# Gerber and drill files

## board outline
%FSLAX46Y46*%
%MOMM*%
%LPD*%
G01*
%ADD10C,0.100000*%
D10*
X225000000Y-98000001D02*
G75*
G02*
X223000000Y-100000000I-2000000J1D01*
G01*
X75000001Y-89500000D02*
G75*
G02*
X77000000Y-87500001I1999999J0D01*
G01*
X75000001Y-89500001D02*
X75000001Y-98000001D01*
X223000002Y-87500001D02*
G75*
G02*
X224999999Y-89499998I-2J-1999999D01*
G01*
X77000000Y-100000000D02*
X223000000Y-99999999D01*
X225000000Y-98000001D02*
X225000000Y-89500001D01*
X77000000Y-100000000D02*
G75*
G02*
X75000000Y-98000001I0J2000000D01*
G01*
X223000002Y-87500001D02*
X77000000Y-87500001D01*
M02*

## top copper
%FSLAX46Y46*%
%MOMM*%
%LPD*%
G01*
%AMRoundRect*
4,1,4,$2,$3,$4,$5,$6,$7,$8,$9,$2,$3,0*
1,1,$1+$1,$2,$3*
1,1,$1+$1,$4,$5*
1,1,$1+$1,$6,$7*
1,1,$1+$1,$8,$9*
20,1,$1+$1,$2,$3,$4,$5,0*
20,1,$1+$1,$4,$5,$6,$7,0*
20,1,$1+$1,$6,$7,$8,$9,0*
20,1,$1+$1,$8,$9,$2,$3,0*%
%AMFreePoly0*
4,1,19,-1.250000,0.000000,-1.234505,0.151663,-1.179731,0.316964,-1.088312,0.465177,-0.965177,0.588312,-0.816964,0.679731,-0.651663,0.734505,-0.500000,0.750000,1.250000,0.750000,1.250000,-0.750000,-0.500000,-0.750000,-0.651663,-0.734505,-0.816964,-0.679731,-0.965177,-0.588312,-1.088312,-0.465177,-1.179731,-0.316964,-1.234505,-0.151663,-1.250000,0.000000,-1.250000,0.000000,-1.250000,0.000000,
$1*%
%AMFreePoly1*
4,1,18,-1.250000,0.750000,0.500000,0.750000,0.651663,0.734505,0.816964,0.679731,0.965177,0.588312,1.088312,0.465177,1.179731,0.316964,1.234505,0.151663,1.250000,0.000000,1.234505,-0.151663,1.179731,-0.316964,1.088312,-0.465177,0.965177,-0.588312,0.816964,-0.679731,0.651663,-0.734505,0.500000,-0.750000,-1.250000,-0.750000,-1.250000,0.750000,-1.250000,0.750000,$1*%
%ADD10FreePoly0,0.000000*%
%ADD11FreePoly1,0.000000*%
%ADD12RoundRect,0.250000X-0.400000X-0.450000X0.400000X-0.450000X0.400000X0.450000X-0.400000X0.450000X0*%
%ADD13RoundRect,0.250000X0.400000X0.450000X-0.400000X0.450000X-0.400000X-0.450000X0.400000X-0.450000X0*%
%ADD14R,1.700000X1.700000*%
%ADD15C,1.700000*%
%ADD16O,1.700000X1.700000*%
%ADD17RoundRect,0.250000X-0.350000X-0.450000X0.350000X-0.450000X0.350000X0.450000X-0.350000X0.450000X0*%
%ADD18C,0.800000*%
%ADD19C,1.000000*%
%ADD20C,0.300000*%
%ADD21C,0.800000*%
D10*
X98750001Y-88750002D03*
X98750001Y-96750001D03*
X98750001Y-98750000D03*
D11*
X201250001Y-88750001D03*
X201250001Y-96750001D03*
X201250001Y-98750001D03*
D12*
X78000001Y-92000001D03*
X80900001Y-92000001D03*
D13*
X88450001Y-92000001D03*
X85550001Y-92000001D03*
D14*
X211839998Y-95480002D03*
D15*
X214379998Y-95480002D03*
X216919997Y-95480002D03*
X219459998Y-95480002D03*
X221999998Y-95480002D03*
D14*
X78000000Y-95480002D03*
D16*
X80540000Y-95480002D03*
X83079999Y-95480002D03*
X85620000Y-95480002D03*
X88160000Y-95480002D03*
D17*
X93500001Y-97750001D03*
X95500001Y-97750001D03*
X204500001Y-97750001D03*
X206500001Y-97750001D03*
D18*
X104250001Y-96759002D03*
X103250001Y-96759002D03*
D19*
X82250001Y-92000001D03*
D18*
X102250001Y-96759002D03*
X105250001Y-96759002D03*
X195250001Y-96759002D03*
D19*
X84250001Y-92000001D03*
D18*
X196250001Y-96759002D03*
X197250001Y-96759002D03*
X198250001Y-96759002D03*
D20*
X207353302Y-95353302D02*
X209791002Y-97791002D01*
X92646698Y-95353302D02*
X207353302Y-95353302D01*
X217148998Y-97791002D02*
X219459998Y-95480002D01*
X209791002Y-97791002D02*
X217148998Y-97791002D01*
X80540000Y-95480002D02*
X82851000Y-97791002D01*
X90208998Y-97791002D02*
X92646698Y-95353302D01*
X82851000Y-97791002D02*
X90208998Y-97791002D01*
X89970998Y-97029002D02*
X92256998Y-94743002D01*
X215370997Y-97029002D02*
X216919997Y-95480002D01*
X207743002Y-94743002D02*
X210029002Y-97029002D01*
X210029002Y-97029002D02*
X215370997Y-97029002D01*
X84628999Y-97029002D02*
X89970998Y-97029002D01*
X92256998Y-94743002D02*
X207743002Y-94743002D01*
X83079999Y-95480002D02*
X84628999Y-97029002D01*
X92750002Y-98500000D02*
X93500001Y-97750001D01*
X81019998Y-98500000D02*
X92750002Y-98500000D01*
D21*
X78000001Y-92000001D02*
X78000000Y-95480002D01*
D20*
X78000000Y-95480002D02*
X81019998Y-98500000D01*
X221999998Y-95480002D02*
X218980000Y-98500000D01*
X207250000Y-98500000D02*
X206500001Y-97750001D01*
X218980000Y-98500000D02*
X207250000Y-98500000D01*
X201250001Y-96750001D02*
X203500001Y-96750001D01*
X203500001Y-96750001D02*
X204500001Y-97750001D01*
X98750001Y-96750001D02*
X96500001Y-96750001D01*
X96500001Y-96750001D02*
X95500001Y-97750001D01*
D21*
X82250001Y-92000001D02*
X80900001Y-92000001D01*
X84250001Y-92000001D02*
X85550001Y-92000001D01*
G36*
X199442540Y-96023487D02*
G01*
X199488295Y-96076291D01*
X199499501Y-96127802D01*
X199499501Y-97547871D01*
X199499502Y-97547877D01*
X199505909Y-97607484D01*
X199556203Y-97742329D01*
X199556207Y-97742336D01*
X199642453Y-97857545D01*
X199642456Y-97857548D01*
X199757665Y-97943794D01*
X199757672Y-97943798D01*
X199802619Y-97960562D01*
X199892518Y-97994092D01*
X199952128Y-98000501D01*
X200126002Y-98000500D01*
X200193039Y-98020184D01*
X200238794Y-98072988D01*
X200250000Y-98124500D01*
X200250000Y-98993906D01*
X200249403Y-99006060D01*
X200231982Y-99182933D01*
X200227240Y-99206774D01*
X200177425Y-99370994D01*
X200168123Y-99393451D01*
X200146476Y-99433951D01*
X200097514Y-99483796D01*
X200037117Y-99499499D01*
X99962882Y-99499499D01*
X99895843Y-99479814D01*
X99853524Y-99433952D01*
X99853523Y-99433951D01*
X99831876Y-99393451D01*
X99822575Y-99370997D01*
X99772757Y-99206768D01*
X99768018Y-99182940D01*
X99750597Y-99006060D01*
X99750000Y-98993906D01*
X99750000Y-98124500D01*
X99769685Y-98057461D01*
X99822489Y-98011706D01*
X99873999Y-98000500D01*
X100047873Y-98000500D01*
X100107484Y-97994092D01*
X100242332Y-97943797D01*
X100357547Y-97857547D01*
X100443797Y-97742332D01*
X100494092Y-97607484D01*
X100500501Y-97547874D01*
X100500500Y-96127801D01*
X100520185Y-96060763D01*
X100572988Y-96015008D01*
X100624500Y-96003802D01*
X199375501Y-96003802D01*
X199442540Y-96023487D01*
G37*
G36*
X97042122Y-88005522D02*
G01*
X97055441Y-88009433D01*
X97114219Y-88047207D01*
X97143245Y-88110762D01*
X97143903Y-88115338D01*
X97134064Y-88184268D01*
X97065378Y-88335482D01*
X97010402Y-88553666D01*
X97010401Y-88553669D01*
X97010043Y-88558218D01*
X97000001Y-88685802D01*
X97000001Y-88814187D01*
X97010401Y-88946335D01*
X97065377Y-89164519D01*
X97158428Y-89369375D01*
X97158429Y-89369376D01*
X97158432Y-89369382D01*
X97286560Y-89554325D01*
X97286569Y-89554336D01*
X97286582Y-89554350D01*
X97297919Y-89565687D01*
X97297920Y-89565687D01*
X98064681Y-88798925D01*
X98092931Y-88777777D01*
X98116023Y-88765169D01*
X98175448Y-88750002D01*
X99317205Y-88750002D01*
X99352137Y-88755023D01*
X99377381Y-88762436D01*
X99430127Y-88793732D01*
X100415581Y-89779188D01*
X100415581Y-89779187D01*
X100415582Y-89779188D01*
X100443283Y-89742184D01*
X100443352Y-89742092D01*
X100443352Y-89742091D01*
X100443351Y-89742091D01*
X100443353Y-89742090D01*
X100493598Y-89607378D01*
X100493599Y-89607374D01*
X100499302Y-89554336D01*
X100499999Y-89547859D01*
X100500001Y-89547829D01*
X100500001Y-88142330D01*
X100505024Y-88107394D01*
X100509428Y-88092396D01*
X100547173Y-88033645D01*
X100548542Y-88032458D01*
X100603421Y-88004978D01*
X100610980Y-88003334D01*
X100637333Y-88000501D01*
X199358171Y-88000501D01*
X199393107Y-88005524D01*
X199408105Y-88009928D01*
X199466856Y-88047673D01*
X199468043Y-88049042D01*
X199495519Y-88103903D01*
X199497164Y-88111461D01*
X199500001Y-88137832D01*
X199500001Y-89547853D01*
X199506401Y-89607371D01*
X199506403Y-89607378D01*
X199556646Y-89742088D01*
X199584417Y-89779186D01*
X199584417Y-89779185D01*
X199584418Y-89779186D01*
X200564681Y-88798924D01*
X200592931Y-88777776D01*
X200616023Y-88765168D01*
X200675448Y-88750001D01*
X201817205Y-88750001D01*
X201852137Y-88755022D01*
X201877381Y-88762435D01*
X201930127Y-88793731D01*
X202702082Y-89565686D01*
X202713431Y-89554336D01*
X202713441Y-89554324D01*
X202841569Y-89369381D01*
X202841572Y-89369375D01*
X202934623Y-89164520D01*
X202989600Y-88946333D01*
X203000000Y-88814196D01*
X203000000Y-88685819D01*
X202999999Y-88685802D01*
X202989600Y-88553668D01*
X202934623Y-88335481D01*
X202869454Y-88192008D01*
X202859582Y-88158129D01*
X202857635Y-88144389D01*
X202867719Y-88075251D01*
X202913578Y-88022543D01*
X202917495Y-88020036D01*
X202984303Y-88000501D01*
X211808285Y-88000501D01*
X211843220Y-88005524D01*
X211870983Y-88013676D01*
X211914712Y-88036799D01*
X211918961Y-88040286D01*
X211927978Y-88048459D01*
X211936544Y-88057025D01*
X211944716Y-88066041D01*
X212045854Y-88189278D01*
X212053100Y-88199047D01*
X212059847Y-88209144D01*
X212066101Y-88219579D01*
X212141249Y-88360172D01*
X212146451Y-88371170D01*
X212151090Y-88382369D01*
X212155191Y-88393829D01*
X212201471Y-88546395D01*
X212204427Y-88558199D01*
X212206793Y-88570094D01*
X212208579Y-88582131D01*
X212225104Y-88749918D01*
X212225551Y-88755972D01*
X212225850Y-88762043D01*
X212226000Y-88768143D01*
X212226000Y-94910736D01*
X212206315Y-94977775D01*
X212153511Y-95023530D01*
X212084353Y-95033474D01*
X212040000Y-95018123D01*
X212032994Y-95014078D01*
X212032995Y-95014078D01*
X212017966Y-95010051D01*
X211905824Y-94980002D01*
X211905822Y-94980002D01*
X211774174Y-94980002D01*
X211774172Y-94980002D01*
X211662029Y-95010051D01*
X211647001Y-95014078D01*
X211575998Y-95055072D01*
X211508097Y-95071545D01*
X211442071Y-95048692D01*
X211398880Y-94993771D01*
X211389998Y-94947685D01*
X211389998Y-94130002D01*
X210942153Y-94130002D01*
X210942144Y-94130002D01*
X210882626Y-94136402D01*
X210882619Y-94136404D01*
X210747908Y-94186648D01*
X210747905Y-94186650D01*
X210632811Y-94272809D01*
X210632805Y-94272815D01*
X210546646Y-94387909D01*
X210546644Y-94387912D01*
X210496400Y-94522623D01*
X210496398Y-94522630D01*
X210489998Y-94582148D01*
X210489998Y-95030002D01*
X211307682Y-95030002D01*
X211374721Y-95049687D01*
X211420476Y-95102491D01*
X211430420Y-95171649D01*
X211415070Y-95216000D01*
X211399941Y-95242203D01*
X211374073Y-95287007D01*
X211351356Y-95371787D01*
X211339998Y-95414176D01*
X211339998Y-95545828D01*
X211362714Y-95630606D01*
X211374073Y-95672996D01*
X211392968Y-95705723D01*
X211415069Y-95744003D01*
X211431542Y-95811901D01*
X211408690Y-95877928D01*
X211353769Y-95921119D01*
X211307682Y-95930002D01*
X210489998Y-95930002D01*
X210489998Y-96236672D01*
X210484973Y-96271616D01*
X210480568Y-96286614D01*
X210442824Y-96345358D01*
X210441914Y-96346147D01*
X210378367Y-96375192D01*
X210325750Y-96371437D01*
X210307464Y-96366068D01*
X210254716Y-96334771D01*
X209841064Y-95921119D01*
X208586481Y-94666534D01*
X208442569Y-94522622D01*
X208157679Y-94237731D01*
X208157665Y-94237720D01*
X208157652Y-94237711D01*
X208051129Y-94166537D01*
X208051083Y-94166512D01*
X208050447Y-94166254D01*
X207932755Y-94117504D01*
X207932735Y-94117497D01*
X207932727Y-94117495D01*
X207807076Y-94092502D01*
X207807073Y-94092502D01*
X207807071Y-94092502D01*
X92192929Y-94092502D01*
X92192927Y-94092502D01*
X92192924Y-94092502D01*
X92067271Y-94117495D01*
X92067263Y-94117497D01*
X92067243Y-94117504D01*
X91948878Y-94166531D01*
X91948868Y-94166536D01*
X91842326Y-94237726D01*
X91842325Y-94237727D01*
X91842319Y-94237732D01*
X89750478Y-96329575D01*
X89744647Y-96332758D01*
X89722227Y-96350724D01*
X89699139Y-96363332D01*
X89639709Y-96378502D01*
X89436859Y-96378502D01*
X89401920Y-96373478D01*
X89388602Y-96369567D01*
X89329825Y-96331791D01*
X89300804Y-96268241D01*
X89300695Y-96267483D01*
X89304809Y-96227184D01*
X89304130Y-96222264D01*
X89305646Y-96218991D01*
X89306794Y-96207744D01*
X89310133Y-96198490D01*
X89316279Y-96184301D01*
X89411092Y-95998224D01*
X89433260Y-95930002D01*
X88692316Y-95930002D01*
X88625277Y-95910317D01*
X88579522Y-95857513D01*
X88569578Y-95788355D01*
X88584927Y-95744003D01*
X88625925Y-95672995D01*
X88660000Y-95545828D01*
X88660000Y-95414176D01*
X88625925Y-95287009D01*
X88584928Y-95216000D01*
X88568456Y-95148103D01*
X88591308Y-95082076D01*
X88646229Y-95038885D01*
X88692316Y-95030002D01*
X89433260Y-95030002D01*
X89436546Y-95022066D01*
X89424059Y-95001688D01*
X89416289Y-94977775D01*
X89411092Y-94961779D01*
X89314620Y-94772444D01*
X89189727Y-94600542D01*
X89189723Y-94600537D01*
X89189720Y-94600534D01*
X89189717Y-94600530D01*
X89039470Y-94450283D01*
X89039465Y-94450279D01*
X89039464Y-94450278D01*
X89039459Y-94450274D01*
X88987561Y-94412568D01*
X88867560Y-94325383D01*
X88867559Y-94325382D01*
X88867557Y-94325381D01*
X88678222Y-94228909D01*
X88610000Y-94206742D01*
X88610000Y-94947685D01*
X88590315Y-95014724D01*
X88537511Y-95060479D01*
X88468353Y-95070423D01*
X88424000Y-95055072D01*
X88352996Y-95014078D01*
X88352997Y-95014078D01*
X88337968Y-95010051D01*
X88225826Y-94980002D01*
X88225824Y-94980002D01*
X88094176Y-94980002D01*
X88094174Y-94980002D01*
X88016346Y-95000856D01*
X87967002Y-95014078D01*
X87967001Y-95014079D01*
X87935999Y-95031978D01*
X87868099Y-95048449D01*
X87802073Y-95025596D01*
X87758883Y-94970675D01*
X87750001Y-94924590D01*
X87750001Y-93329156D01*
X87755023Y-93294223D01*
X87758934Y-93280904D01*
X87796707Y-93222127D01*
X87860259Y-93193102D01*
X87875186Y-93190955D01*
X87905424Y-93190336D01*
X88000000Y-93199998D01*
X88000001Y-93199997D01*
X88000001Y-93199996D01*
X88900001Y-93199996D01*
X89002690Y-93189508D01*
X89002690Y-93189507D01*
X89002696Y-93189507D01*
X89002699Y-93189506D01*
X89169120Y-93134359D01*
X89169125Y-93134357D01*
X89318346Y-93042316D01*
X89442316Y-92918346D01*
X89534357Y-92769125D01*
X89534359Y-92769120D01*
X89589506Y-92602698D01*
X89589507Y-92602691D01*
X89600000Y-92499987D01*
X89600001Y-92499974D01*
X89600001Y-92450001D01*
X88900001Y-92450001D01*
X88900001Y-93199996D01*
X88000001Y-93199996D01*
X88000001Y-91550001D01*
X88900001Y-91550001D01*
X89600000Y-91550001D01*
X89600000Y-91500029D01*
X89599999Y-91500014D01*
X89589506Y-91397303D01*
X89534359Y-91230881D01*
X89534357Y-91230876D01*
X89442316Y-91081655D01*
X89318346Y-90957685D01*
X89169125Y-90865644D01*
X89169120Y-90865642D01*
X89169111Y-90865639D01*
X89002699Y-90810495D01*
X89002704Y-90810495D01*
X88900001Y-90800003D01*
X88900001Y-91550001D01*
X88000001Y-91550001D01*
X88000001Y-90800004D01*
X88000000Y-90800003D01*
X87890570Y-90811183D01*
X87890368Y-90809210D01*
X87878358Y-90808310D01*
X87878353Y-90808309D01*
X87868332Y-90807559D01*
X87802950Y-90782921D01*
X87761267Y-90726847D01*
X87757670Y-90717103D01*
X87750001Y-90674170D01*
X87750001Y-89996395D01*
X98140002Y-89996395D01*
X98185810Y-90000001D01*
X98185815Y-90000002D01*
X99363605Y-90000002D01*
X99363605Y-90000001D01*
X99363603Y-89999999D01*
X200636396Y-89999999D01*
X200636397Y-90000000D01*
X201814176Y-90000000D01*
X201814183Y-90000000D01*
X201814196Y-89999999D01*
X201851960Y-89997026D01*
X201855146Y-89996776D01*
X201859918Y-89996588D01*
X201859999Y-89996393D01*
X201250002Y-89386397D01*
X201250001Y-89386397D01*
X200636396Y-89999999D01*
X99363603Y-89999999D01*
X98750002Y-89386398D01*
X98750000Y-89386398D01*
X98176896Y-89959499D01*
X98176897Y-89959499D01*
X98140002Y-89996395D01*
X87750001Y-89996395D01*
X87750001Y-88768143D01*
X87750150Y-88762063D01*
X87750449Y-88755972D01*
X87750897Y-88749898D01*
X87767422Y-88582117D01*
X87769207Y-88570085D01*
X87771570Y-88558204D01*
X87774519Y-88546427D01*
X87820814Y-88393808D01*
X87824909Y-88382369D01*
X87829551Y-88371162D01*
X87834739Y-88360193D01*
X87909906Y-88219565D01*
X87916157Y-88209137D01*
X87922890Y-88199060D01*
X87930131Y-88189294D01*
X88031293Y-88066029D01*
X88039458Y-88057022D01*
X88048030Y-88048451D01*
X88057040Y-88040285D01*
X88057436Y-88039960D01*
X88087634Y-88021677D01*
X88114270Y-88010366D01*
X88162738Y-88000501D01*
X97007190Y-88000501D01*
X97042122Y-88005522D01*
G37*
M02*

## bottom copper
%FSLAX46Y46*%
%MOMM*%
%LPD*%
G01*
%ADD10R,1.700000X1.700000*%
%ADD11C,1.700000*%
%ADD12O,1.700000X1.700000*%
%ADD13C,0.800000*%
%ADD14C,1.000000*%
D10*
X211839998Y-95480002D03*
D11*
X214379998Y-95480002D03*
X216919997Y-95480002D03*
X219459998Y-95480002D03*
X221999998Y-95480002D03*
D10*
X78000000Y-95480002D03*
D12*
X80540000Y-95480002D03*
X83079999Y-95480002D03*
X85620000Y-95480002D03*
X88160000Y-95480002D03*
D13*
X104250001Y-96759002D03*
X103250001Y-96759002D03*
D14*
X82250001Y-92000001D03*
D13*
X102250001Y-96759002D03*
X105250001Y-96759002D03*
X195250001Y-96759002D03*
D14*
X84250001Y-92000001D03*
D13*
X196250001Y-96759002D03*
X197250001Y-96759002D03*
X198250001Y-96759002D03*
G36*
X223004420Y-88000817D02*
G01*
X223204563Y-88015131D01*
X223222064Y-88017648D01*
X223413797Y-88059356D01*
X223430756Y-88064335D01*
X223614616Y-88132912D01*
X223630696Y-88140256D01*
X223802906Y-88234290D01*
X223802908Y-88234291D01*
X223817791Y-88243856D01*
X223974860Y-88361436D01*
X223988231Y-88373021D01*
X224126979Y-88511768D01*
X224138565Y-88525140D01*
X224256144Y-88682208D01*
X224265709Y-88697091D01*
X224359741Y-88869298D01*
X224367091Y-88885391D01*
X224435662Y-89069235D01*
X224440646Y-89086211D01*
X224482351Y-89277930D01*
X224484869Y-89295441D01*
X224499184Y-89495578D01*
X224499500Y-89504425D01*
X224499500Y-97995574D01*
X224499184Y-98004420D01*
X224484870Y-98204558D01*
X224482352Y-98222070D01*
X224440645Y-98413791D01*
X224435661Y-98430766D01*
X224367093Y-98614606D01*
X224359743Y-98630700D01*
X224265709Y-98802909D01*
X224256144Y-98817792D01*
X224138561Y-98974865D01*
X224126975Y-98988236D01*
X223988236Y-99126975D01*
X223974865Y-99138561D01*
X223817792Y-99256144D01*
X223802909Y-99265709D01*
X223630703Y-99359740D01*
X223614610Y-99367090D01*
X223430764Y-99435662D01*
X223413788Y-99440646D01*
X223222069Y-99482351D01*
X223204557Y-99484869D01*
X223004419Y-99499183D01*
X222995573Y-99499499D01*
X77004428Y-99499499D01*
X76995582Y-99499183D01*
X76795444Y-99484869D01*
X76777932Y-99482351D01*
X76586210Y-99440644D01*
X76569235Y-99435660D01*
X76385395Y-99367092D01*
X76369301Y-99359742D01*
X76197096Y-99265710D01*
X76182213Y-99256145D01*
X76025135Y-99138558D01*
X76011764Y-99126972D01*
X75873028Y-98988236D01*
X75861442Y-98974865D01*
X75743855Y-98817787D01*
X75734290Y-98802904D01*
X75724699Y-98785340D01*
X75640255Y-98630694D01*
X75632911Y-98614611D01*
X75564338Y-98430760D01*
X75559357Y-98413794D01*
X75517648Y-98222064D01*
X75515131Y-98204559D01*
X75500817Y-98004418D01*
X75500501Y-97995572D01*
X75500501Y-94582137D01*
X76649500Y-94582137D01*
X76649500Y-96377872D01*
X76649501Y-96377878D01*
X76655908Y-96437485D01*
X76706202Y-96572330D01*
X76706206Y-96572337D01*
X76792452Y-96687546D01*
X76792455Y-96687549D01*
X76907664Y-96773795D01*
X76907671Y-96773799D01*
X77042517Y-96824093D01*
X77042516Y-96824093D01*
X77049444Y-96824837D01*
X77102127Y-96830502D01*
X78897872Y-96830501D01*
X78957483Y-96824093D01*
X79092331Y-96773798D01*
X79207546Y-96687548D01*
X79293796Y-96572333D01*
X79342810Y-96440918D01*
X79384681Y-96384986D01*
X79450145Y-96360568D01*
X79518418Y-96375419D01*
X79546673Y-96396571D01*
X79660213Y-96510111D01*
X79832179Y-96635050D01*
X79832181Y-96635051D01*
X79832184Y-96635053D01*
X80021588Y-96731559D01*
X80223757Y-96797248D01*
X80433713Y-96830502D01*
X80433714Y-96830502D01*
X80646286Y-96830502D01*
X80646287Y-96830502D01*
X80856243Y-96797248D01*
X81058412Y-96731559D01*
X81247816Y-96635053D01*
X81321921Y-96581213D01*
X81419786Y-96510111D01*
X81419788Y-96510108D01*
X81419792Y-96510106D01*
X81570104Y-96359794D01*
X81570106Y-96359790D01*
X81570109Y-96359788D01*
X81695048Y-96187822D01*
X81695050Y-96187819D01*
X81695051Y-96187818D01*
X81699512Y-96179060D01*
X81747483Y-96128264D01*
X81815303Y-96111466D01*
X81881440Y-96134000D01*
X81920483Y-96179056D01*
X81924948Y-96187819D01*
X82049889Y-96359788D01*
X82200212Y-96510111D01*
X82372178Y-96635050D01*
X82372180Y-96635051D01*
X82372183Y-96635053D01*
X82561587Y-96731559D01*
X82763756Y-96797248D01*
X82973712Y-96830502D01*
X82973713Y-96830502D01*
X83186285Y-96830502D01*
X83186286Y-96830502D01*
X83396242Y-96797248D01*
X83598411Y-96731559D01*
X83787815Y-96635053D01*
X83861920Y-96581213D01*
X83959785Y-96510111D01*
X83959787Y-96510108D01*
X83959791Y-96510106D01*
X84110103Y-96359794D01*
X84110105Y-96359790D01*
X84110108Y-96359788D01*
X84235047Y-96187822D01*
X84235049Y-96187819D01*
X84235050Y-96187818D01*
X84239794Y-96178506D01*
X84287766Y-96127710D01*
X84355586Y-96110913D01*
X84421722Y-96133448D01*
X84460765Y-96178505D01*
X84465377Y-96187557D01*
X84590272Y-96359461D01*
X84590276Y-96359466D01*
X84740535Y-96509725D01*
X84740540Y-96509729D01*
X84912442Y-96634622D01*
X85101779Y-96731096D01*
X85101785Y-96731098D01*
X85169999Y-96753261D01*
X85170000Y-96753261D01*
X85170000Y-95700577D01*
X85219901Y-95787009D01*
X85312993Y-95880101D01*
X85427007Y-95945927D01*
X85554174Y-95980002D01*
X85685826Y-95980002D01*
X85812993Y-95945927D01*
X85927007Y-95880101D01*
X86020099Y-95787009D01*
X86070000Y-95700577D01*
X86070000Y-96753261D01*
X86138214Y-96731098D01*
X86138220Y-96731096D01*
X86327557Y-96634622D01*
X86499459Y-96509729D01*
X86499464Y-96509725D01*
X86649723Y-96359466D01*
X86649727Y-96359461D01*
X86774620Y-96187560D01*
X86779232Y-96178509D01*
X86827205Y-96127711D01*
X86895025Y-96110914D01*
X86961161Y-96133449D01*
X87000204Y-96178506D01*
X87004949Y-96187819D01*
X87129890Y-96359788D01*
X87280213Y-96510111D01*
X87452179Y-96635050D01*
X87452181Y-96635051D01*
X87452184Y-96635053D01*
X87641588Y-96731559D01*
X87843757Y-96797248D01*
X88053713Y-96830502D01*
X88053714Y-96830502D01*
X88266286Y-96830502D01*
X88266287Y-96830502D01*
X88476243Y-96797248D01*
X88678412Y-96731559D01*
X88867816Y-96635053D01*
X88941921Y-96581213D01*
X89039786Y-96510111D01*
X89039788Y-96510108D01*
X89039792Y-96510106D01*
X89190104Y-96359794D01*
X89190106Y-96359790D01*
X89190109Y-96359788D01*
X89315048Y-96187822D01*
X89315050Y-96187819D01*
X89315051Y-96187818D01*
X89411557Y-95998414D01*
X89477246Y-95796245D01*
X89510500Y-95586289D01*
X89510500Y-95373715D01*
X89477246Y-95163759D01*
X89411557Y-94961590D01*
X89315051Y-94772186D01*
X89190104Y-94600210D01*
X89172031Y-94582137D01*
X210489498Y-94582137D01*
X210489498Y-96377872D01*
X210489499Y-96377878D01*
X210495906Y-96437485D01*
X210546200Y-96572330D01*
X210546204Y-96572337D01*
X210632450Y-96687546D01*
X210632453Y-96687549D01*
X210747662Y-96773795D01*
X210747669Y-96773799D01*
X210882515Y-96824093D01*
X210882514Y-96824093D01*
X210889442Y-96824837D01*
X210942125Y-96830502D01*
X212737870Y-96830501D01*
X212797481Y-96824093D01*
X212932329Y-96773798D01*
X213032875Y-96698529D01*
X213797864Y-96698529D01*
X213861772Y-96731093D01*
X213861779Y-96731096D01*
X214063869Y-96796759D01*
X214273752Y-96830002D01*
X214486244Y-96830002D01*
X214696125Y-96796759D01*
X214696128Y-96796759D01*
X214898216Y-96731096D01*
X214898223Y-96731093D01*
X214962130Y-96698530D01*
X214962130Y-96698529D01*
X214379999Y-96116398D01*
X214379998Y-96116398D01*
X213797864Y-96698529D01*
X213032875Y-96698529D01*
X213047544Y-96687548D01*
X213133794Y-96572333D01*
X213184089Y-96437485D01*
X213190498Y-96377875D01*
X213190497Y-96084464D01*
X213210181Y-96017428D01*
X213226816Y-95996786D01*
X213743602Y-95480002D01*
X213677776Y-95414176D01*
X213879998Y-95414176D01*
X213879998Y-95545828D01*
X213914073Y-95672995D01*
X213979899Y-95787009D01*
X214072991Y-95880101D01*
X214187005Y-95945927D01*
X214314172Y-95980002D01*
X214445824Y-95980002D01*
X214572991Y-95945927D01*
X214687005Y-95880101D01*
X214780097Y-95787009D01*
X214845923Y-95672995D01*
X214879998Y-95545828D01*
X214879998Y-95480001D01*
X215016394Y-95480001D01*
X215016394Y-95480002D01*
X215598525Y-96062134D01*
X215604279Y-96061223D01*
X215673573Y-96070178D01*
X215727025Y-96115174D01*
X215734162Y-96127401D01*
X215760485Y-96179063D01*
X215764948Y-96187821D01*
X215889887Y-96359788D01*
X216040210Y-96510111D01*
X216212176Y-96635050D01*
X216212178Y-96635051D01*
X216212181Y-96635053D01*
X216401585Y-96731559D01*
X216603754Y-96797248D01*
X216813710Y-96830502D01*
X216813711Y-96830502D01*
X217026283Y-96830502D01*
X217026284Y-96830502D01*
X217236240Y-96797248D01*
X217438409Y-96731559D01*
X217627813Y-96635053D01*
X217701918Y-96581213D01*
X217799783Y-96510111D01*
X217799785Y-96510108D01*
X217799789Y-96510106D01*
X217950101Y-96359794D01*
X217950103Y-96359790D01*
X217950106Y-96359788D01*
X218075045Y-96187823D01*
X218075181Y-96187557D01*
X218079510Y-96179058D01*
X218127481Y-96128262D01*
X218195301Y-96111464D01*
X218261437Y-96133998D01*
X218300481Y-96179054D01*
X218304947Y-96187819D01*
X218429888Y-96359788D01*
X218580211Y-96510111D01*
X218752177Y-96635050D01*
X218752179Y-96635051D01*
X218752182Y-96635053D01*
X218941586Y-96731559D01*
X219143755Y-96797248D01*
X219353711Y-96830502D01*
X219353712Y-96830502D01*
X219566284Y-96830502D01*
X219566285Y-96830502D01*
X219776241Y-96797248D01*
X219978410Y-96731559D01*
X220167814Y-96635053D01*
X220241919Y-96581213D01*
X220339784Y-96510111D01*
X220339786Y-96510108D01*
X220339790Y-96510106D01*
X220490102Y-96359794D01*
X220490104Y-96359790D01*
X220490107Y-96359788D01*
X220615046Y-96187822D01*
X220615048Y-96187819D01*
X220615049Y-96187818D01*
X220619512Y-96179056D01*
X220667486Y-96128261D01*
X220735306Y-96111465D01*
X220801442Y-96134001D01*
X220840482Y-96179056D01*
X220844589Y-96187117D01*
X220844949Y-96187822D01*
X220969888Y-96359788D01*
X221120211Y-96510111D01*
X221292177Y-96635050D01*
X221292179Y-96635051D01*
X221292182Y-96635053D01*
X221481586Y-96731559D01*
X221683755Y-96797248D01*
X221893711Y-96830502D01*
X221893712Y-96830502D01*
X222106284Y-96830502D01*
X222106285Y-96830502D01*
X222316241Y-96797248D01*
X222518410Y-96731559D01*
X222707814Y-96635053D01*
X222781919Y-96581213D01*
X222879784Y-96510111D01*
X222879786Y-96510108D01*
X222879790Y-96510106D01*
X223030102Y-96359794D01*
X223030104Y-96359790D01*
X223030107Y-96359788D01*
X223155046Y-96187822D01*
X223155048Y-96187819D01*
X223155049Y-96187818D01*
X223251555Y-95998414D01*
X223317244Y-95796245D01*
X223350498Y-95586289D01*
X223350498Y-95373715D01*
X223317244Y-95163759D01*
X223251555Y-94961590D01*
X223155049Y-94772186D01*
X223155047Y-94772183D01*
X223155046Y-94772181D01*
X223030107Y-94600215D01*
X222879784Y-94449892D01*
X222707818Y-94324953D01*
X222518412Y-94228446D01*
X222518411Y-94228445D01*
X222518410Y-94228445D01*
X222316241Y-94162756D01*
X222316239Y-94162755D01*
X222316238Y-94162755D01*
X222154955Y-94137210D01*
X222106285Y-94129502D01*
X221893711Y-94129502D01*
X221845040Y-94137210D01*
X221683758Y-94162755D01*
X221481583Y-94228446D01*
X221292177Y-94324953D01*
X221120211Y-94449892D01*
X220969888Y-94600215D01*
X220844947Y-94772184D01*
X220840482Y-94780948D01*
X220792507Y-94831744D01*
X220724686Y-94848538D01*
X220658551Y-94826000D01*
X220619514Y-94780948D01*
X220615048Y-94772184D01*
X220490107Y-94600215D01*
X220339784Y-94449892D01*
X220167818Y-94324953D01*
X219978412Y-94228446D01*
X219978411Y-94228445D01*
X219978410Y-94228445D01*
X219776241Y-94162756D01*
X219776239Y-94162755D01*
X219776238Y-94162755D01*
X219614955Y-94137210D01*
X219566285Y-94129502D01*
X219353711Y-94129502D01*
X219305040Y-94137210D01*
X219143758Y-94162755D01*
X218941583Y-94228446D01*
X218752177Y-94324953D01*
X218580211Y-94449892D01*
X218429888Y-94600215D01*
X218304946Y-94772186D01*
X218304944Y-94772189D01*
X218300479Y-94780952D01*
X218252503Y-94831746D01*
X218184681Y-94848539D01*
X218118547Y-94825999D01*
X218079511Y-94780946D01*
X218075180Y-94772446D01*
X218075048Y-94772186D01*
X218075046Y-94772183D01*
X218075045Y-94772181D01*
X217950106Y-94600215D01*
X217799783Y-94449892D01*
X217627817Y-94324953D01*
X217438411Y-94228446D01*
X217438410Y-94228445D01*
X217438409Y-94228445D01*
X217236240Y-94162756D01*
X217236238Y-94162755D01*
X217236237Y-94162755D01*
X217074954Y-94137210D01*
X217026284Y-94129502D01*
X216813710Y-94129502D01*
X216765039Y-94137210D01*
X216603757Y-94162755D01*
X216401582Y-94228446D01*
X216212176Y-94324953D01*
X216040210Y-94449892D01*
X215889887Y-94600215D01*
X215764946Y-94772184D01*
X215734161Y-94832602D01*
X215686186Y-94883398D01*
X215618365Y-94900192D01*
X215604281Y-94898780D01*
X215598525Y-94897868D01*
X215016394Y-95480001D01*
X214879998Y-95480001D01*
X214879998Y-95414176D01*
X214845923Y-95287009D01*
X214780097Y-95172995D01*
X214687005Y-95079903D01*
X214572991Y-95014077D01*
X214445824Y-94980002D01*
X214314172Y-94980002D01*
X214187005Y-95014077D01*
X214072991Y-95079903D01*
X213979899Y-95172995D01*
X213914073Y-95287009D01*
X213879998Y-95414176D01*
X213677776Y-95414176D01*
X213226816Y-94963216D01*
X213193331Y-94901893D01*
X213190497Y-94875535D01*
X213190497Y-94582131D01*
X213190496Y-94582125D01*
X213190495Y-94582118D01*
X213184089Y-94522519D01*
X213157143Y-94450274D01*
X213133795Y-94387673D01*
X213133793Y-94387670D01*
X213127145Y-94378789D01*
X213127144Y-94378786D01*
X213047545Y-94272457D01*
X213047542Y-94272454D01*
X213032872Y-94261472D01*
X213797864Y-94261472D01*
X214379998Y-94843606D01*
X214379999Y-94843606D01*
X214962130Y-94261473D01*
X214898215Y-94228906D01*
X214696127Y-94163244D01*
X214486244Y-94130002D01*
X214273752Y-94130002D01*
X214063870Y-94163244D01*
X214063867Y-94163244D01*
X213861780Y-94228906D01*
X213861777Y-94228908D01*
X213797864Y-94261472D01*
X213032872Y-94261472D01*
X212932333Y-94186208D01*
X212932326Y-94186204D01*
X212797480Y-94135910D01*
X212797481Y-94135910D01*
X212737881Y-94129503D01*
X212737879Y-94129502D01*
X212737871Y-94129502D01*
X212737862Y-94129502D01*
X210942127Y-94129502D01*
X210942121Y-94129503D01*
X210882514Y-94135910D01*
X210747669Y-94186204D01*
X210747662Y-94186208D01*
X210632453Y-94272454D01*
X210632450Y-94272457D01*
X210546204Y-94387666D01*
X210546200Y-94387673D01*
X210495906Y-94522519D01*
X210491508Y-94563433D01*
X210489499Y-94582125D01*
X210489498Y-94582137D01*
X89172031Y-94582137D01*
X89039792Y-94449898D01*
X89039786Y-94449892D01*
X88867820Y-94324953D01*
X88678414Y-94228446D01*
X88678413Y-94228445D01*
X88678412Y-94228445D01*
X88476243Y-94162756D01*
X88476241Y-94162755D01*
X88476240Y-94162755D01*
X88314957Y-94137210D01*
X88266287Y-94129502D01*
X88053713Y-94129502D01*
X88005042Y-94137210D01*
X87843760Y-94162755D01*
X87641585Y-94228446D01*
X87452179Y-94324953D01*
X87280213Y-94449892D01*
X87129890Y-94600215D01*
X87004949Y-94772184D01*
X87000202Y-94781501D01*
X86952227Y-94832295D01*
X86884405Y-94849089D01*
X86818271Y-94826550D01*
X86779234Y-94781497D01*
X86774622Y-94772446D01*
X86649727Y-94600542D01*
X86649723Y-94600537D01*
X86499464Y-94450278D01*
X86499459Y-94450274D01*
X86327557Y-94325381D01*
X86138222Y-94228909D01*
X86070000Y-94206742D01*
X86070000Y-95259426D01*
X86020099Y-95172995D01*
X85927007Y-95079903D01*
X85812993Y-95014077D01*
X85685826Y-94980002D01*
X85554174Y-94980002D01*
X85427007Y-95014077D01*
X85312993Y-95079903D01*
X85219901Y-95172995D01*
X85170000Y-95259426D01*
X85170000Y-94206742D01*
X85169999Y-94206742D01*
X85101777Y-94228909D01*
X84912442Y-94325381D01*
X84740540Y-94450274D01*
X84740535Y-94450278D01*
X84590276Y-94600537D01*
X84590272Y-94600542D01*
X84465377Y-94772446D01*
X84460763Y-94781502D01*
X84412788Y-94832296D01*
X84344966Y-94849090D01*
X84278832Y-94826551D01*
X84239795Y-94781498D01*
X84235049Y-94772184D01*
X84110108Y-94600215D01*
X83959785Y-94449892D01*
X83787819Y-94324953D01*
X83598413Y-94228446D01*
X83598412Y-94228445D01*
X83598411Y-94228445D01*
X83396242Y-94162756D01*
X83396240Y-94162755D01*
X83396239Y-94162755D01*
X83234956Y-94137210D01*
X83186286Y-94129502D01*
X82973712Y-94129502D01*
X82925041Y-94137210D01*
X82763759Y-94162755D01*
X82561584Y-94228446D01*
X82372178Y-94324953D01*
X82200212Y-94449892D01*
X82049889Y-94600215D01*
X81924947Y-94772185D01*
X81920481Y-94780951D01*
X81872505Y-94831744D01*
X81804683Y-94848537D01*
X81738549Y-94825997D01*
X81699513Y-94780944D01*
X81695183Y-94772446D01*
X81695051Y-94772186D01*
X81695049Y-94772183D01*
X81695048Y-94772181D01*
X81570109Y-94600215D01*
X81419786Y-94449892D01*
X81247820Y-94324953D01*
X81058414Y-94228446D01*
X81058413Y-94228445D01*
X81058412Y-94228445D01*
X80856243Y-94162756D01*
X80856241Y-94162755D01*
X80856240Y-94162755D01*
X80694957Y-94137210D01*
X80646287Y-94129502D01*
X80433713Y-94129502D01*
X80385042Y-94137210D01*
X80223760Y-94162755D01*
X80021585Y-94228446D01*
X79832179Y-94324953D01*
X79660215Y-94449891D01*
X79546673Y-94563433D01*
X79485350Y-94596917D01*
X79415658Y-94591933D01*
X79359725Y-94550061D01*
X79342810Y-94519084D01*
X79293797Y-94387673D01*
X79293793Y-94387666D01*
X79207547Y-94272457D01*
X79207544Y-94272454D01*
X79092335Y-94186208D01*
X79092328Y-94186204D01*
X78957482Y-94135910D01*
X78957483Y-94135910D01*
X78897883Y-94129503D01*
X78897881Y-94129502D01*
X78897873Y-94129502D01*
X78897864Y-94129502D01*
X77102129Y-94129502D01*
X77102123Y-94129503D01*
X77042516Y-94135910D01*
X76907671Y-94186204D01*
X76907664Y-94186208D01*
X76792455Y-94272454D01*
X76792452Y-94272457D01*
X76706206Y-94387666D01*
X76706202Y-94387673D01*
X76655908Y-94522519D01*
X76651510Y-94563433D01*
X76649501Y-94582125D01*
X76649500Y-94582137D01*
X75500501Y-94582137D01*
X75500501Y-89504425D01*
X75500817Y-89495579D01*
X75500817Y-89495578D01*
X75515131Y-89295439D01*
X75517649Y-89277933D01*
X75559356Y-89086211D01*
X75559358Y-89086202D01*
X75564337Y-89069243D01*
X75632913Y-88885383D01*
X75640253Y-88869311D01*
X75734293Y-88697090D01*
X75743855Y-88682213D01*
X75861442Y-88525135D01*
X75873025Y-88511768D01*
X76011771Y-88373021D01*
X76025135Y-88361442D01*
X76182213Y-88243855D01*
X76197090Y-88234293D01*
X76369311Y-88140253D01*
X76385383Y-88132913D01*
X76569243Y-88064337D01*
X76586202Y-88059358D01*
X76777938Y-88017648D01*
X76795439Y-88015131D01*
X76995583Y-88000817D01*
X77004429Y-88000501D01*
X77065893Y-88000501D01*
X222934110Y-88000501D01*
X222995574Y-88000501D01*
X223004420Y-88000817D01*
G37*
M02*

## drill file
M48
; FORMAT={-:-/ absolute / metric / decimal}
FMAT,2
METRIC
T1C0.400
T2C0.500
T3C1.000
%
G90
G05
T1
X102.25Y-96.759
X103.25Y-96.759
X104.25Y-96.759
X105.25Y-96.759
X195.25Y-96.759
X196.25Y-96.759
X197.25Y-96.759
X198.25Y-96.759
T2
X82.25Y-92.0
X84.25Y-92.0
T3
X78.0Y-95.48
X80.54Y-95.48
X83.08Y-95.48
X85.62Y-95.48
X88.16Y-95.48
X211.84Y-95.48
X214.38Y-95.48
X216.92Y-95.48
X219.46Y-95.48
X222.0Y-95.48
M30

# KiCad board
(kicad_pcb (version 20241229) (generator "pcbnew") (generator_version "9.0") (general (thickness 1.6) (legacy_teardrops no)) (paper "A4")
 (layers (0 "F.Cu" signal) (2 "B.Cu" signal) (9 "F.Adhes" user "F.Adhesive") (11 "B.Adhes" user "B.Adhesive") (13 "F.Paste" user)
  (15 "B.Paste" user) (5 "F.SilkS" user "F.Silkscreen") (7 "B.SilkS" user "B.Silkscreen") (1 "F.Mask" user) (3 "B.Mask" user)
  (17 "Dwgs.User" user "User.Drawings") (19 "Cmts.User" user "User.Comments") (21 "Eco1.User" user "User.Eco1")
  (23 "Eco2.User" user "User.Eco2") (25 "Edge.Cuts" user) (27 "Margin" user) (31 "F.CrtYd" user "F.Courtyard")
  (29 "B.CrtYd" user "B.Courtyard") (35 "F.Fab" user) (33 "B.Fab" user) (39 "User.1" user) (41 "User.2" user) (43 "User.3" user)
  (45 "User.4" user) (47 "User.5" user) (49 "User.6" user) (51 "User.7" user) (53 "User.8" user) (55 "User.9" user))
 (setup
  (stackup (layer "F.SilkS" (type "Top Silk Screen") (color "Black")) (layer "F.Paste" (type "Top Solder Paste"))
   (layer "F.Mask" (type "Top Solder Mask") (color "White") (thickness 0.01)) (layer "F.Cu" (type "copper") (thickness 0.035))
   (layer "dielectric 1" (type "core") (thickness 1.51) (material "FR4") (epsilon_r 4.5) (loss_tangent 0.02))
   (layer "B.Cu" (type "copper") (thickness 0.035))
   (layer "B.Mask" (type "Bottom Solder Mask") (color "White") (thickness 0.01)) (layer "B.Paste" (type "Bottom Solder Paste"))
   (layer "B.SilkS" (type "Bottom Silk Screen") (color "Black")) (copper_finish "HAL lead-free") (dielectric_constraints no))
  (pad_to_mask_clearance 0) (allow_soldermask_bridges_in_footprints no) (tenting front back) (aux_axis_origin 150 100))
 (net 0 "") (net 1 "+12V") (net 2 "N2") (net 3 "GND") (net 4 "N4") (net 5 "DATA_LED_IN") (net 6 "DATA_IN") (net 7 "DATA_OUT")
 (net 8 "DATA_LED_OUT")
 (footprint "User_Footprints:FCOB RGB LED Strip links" (layer "F.Cu") (at 100.000001 93.750001)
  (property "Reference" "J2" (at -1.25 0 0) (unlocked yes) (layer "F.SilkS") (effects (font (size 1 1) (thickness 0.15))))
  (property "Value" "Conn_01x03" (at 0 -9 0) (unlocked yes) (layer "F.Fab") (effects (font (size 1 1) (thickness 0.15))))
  (pad "1" smd roundrect (at -1.25 -4.999999) (size 2.5 1.5) (layers "F.Cu" "F.Mask" "F.Paste") (roundrect_rratio 0.5) (chamfer_ratio 0)
   (chamfer top_right bottom_right) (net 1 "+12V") (thermal_bridge_angle 45))
  (pad "2" smd roundrect (at -1.25 3) (size 2.5 1.5) (layers "F.Cu" "F.Mask" "F.Paste") (roundrect_rratio 0.5) (chamfer_ratio 0)
   (chamfer top_right bottom_right) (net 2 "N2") (thermal_bridge_angle 45))
  (pad "3" smd roundrect (at -1.25 4.999999) (size 2.5 1.5) (layers "F.Cu" "F.Mask" "F.Paste") (roundrect_rratio 0.5) (chamfer_ratio 0)
   (chamfer top_right bottom_right) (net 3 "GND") (thermal_bridge_angle 45)))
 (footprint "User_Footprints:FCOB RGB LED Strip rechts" (layer "F.Cu") (at 200.000001 93.750001)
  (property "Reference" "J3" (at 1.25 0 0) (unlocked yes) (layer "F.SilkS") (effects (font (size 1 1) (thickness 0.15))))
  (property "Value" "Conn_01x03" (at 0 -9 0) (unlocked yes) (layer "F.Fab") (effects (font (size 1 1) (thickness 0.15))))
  (pad "1" smd roundrect (at 1.25 -5) (size 2.5 1.5) (layers "F.Cu" "F.Mask" "F.Paste") (roundrect_rratio 0.5) (chamfer_ratio 0)
   (chamfer top_left bottom_left) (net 1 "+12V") (thermal_bridge_angle 45))
  (pad "2" smd roundrect (at 1.25 3) (size 2.5 1.5) (layers "F.Cu" "F.Mask" "F.Paste") (roundrect_rratio 0.5) (chamfer_ratio 0)
   (chamfer top_left bottom_left) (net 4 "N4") (thermal_bridge_angle 45))
  (pad "3" smd roundrect (at 1.25 5) (size 2.5 1.5) (layers "F.Cu" "F.Mask" "F.Paste") (roundrect_rratio 0.5) (chamfer_ratio 0)
   (chamfer top_left bottom_left) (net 3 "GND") (thermal_bridge_angle 45)))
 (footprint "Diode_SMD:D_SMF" (layer "F.Cu") (at 79.450001 92.000001)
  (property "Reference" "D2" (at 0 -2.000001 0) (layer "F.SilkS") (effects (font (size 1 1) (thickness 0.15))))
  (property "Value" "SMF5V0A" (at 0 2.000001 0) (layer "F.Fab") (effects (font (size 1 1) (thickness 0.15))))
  (pad "1" smd roundrect (at -1.45 0) (size 1.3 1.4) (layers "F.Cu" "F.Mask" "F.Paste") (roundrect_rratio 0.1923076923)
   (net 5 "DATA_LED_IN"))
  (pad "2" smd roundrect (at 1.45 0) (size 1.3 1.4) (layers "F.Cu" "F.Mask" "F.Paste") (roundrect_rratio 0.1923076923) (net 3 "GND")))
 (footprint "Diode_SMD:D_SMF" (layer "F.Cu") (at 87.000001 92.000001 180)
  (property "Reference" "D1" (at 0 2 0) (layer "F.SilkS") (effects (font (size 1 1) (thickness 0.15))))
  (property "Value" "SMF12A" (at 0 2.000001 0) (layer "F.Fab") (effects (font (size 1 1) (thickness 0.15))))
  (pad "1" smd roundrect (at -1.45 0 180) (size 1.3 1.4) (layers "F.Cu" "F.Mask" "F.Paste") (roundrect_rratio 0.1923076923) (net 1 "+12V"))
  (pad "2" smd roundrect (at 1.45 0 180) (size 1.3 1.4) (layers "F.Cu" "F.Mask" "F.Paste") (roundrect_rratio 0.1923076923) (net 3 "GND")))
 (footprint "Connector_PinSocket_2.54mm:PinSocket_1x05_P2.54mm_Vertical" (layer "F.Cu") (at 211.839998 95.480002 90)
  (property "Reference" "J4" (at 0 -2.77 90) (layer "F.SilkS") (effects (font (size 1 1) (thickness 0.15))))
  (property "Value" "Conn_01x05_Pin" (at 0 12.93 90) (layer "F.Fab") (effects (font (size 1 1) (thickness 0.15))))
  (pad "1" thru_hole rect (at 0 0 90) (size 1.7 1.7) (drill 1) (layers "*.Cu" "*.Mask") (remove_unused_layers no) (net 1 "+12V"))
  (pad "2" thru_hole circle (at 0 2.54 90) (size 1.7 1.7) (drill 1) (layers "*.Cu" "*.Mask") (remove_unused_layers no) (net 3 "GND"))
  (pad "3" thru_hole circle (at 0 5.079999 90) (size 1.7 1.7) (drill 1) (layers "*.Cu" "*.Mask") (remove_unused_layers no) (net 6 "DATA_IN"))
  (pad "4" thru_hole circle (at 0 7.62 90) (size 1.7 1.7) (drill 1) (layers "*.Cu" "*.Mask") (remove_unused_layers no) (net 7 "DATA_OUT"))
  (pad "5" thru_hole circle (at 0 10.16 90) (size 1.7 1.7) (drill 1) (layers "*.Cu" "*.Mask") (remove_unused_layers no)
   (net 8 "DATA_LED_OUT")))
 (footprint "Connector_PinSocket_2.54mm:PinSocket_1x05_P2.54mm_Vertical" (layer "F.Cu") (at 78 95.480002 90)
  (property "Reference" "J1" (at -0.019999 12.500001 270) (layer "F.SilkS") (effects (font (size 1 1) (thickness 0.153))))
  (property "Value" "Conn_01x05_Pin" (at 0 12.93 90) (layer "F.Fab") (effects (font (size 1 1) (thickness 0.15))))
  (pad "1" thru_hole rect (at 0 0 90) (size 1.7 1.7) (drill 1) (layers "*.Cu" "*.Mask") (remove_unused_layers no) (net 5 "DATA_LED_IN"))
  (pad "2" thru_hole oval (at 0 2.54 90) (size 1.7 1.7) (drill 1) (layers "*.Cu" "*.Mask") (remove_unused_layers no) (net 7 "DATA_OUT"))
  (pad "3" thru_hole oval (at 0 5.079999 90) (size 1.7 1.7) (drill 1) (layers "*.Cu" "*.Mask") (remove_unused_layers no) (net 6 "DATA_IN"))
  (pad "4" thru_hole oval (at 0 7.62 90) (size 1.7 1.7) (drill 1) (layers "*.Cu" "*.Mask") (remove_unused_layers no) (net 3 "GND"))
  (pad "5" thru_hole oval (at 0 10.16 90) (size 1.7 1.7) (drill 1) (layers "*.Cu" "*.Mask") (remove_unused_layers no) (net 1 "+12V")))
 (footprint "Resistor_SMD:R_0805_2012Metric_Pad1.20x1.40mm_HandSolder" (layer "F.Cu") (at 94.500001 97.750001)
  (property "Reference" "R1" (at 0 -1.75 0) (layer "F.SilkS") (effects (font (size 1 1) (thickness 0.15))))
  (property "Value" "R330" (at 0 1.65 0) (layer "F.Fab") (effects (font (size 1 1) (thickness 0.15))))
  (pad "1" smd roundrect (at -1 0) (size 1.2 1.4) (layers "F.Cu" "F.Mask" "F.Paste") (roundrect_rratio 0.208333) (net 5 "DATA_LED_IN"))
  (pad "2" smd roundrect (at 1 0) (size 1.2 1.4) (layers "F.Cu" "F.Mask" "F.Paste") (roundrect_rratio 0.208333) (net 2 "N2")))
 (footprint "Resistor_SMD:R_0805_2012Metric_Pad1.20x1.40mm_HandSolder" (layer "F.Cu") (at 205.500001 97.750001)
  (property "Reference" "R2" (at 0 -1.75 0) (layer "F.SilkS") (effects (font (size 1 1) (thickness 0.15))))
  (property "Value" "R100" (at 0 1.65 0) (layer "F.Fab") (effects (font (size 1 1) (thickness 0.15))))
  (pad "1" smd roundrect (at -1 0) (size 1.2 1.4) (layers "F.Cu" "F.Mask" "F.Paste") (roundrect_rratio 0.208333) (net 4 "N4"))
  (pad "2" smd roundrect (at 1 0) (size 1.2 1.4) (layers "F.Cu" "F.Mask" "F.Paste") (roundrect_rratio 0.208333) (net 8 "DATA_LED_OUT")))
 (gr_arc (start 225 98.000001) (mid 224.414214 99.414215) (end 223 99.999999) (stroke (width 0.1) (type default)) (layer "Edge.Cuts"))
 (gr_arc (start 75.000001 89.5) (mid 75.585788 88.085788) (end 77 87.500001) (stroke (width 0.1) (type default)) (layer "Edge.Cuts"))
 (gr_line (start 75.000001 89.500001) (end 75.000001 98.000001) (stroke (width 0.1) (type default)) (layer "Edge.Cuts"))
 (gr_arc (start 223.000002 87.500001) (mid 224.414214 88.085787) (end 225 89.499998) (stroke (width 0.1) (type default)) (layer "Edge.Cuts"))
 (gr_line (start 77 100) (end 223 99.999999) (stroke (width 0.1) (type default)) (layer "Edge.Cuts"))
 (gr_line (start 225 98.000001) (end 225 89.500001) (stroke (width 0.1) (type default)) (layer "Edge.Cuts"))
 (gr_arc (start 77 100) (mid 75.585788 99.414213) (end 75.000001 98.000001) (stroke (width 0.1) (type default)) (layer "Edge.Cuts"))
 (gr_line (start 223.000002 87.500001) (end 77 87.500001) (stroke (width 0.1) (type default)) (layer "Edge.Cuts"))
 (segment (start 207.353302 95.353302) (end 209.791002 97.791002) (width 0.3) (layer "F.Cu") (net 7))
 (segment (start 92.646698 95.353302) (end 207.353302 95.353302) (width 0.3) (layer "F.Cu") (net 7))
 (segment (start 217.148998 97.791002) (end 219.459998 95.480002) (width 0.3) (layer "F.Cu") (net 7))
 (segment (start 209.791002 97.791002) (end 217.148998 97.791002) (width 0.3) (layer "F.Cu") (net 7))
 (segment (start 80.54 95.480002) (end 82.851 97.791002) (width 0.3) (layer "F.Cu") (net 7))
 (segment (start 90.208998 97.791002) (end 92.646698 95.353302) (width 0.3) (layer "F.Cu") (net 7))
 (segment (start 82.851 97.791002) (end 90.208998 97.791002) (width 0.3) (layer "F.Cu") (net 7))
 (segment (start 89.970998 97.029002) (end 92.256998 94.743002) (width 0.3) (layer "F.Cu") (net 6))
 (segment (start 215.370997 97.029002) (end 216.919997 95.480002) (width 0.3) (layer "F.Cu") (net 6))
 (segment (start 207.743002 94.743002) (end 210.029002 97.029002) (width 0.3) (layer "F.Cu") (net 6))
 (segment (start 210.029002 97.029002) (end 215.370997 97.029002) (width 0.3) (layer "F.Cu") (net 6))
 (segment (start 84.628999 97.029002) (end 89.970998 97.029002) (width 0.3) (layer "F.Cu") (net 6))
 (segment (start 92.256998 94.743002) (end 207.743002 94.743002) (width 0.3) (layer "F.Cu") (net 6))
 (segment (start 83.079999 95.480002) (end 84.628999 97.029002) (width 0.3) (layer "F.Cu") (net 6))
 (segment (start 92.750002 98.5) (end 93.500001 97.750001) (width 0.3) (layer "F.Cu") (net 5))
 (segment (start 81.019998 98.5) (end 92.750002 98.5) (width 0.3) (layer "F.Cu") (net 5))
 (segment (start 78.000001 92.000001) (end 78 95.480002) (width 0.8) (layer "F.Cu") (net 5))
 (segment (start 78 95.480002) (end 81.019998 98.5) (width 0.3) (layer "F.Cu") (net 5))
 (segment (start 221.999998 95.480002) (end 218.98 98.5) (width 0.3) (layer "F.Cu") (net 8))
 (segment (start 207.25 98.5) (end 206.500001 97.750001) (width 0.3) (layer "F.Cu") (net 8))
 (segment (start 218.98 98.5) (end 207.25 98.5) (width 0.3) (layer "F.Cu") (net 8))
 (segment (start 201.250001 96.750001) (end 203.500001 96.750001) (width 0.3) (layer "F.Cu") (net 4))
 (segment (start 203.500001 96.750001) (end 204.500001 97.750001) (width 0.3) (layer "F.Cu") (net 4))
 (segment (start 98.750001 96.750001) (end 96.500001 96.750001) (width 0.3) (layer "F.Cu") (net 2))
 (segment (start 96.500001 96.750001) (end 95.500001 97.750001) (width 0.3) (layer "F.Cu") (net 2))
 (segment (start 82.250001 92.000001) (end 80.900001 92.000001) (width 0.8) (layer "F.Cu") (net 3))
 (segment (start 84.250001 92.000001) (end 85.550001 92.000001) (width 0.8) (layer "F.Cu") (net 3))
 (via (at 104.250001 96.759002) (size 0.8) (drill 0.4) (layers "F.Cu" "B.Cu") (free yes) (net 3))
 (via (at 103.250001 96.759002) (size 0.8) (drill 0.4) (layers "F.Cu" "B.Cu") (free yes) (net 3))
 (via (at 82.250001 92.000001) (size 1) (drill 0.5) (layers "F.Cu" "B.Cu") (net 3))
 (via (at 102.250001 96.759002) (size 0.8) (drill 0.4) (layers "F.Cu" "B.Cu") (free yes) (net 3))
 (via (at 105.250001 96.759002) (size 0.8) (drill 0.4) (layers "F.Cu" "B.Cu") (free yes) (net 3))
 (via (at 195.250001 96.759002) (size 0.8) (drill 0.4) (layers "F.Cu" "B.Cu") (free yes) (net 3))
 (via (at 84.250001 92.000001) (size 1) (drill 0.5) (layers "F.Cu" "B.Cu") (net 3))
 (via (at 196.250001 96.759002) (size 0.8) (drill 0.4) (layers "F.Cu" "B.Cu") (free yes) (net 3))
 (via (at 197.250001 96.759002) (size 0.8) (drill 0.4) (layers "F.Cu" "B.Cu") (free yes) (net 3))
 (via (at 198.250001 96.759002) (size 0.8) (drill 0.4) (layers "F.Cu" "B.Cu") (free yes) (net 3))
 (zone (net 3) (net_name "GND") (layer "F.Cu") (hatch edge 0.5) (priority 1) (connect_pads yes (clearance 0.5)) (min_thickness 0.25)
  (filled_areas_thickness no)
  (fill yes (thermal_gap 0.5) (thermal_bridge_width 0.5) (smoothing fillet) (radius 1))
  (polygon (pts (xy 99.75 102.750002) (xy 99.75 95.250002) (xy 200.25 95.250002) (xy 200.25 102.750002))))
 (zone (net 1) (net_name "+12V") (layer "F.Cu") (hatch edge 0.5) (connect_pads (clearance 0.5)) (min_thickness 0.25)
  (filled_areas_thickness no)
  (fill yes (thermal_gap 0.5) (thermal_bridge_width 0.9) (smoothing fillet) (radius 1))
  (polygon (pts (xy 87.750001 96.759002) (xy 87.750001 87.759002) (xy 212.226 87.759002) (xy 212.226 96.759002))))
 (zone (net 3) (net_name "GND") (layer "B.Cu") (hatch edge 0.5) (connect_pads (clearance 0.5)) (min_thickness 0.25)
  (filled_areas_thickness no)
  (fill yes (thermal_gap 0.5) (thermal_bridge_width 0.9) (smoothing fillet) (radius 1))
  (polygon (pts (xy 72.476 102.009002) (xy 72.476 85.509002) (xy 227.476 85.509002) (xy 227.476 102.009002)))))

